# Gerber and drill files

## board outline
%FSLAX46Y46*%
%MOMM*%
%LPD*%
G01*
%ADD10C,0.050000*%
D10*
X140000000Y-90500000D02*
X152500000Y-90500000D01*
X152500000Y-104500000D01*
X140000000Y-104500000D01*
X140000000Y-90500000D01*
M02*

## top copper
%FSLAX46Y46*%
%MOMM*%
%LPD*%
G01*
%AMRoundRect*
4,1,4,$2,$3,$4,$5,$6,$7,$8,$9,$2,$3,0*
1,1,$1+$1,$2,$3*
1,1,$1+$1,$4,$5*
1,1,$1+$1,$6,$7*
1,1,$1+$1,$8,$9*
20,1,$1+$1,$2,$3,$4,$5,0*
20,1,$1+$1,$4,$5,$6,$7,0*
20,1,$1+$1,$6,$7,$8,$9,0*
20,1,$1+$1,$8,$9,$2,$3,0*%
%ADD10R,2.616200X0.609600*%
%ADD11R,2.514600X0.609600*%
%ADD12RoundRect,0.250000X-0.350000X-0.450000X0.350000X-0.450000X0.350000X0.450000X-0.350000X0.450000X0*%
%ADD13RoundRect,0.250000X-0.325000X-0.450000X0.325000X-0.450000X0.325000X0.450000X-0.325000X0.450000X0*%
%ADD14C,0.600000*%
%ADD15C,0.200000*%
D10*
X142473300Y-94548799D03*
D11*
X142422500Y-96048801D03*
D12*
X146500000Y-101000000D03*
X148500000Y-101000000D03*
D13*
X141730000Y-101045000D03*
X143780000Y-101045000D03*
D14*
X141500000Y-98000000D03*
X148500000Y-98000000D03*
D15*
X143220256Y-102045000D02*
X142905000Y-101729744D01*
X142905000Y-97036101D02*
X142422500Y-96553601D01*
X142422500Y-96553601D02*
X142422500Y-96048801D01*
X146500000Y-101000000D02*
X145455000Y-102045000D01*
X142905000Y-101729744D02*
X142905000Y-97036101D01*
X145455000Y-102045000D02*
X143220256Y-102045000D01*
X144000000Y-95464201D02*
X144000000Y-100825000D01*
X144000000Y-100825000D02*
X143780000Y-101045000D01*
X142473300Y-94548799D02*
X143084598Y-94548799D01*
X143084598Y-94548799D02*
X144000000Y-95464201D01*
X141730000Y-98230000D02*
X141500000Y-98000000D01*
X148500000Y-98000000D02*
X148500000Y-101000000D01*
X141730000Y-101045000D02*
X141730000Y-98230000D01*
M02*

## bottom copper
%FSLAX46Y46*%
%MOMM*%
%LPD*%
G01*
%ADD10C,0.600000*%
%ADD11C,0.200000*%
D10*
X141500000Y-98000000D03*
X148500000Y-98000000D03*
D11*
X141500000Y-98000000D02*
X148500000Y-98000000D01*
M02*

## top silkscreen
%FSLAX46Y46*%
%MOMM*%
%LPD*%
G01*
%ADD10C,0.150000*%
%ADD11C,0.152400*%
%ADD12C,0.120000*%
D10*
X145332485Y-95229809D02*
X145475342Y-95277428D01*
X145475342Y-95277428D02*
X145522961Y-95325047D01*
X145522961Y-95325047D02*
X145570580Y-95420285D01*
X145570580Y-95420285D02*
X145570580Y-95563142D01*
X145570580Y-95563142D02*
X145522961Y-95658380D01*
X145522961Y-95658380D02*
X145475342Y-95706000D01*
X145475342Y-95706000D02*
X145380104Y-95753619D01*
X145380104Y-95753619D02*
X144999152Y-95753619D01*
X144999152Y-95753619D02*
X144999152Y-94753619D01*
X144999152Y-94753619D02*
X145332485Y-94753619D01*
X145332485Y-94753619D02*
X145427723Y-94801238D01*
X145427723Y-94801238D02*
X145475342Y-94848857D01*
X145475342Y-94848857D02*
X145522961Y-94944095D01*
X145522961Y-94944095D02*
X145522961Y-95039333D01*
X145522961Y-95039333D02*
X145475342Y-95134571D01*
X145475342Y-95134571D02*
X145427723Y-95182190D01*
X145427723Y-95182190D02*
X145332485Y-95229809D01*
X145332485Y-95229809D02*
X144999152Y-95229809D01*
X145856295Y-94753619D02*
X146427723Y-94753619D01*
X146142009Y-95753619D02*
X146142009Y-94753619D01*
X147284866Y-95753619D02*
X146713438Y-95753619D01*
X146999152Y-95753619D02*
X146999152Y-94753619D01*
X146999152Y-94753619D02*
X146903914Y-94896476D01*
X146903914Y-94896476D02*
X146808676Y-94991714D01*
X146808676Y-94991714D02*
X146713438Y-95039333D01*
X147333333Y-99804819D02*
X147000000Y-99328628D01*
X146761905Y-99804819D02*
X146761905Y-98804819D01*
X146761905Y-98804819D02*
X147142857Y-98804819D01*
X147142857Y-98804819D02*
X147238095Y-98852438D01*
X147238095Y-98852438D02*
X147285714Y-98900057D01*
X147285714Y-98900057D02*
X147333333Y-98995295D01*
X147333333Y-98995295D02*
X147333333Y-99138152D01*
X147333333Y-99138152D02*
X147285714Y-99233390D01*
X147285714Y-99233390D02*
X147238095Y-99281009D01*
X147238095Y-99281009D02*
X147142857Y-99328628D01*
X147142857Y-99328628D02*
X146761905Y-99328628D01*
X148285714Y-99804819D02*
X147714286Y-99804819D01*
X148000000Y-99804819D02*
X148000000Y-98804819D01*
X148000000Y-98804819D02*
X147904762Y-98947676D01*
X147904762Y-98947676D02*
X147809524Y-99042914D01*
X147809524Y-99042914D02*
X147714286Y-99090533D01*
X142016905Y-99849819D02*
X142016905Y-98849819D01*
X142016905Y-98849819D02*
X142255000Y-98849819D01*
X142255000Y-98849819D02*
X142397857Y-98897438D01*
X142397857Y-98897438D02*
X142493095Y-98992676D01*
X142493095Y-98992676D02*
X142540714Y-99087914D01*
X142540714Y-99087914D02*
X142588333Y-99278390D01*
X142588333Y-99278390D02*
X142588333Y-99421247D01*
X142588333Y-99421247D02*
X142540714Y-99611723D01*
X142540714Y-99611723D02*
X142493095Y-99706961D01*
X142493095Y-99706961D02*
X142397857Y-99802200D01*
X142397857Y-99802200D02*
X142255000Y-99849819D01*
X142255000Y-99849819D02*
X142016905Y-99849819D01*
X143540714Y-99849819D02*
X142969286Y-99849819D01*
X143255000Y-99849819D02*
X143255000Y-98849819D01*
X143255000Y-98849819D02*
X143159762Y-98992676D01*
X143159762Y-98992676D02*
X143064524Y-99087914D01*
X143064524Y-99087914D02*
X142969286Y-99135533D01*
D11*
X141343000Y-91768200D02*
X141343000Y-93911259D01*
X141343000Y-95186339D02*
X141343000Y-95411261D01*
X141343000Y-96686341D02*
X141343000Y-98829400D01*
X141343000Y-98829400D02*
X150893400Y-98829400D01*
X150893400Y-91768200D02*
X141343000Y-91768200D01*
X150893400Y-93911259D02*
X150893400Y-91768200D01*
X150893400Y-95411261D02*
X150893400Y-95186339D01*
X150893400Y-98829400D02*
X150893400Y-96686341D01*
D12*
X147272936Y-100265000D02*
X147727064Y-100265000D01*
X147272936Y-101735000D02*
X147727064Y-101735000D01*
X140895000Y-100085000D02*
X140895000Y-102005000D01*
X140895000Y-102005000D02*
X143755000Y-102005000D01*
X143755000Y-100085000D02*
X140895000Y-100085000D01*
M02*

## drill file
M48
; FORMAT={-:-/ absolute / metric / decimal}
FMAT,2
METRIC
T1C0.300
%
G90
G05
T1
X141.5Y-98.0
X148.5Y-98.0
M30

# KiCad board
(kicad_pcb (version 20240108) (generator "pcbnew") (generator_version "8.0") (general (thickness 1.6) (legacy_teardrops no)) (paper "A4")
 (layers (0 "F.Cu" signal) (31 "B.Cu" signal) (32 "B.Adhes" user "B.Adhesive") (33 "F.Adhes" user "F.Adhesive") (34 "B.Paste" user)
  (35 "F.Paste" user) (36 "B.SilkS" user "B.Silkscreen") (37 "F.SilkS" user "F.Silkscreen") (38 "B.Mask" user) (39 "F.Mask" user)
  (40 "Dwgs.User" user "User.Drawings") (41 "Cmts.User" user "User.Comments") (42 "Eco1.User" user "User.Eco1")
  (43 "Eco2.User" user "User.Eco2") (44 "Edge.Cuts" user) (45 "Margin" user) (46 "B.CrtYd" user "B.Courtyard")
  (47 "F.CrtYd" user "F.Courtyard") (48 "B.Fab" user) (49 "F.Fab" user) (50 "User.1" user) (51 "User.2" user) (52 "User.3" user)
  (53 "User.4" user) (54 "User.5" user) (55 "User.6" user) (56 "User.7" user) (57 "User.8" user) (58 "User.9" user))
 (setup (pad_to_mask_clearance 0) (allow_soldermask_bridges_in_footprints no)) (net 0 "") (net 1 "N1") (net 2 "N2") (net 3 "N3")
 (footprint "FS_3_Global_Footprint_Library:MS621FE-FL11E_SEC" (layer "F.Cu") (at 146.1182 95.2988)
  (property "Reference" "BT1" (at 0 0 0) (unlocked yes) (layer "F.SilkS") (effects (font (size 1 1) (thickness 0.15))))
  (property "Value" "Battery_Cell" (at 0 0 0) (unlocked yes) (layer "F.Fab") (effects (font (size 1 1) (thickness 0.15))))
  (fp_line (start -4.7752 -3.5306) (end -4.7752 -1.387541) (stroke (width 0.1524) (type solid)) (layer "F.SilkS"))
  (fp_line (start -4.7752 -0.112461) (end -4.7752 0.112461) (stroke (width 0.1524) (type solid)) (layer "F.SilkS"))
  (fp_line (start -4.7752 1.387541) (end -4.7752 3.5306) (stroke (width 0.1524) (type solid)) (layer "F.SilkS"))
  (fp_line (start -4.7752 3.5306) (end 4.7752 3.5306) (stroke (width 0.1524) (type solid)) (layer "F.SilkS"))
  (fp_line (start 4.7752 -3.5306) (end -4.7752 -3.5306) (stroke (width 0.1524) (type solid)) (layer "F.SilkS"))
  (fp_line (start 4.7752 -1.387541) (end 4.7752 -3.5306) (stroke (width 0.1524) (type solid)) (layer "F.SilkS"))
  (fp_line (start 4.7752 0.112461) (end 4.7752 -0.112461) (stroke (width 0.1524) (type solid)) (layer "F.SilkS"))
  (fp_line (start 4.7752 3.5306) (end 4.7752 1.387541) (stroke (width 0.1524) (type solid)) (layer "F.SilkS"))
  (pad "1" smd rect (at -3.6449 -0.750001) (size 2.6162 0.6096) (layers "F.Cu" "F.Paste" "F.Mask") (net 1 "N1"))
  (pad "2" smd rect (at -3.6957 0.750001) (size 2.5146 0.6096) (layers "F.Cu" "F.Paste" "F.Mask") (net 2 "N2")))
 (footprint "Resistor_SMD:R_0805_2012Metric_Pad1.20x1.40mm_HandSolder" (layer "F.Cu") (at 147.5 101)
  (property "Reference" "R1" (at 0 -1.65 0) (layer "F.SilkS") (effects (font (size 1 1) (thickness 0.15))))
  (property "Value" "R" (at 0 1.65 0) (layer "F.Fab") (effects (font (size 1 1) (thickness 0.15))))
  (fp_line (start -0.227064 -0.735) (end 0.227064 -0.735) (stroke (width 0.12) (type solid)) (layer "F.SilkS"))
  (fp_line (start -0.227064 0.735) (end 0.227064 0.735) (stroke (width 0.12) (type solid)) (layer "F.SilkS"))
  (pad "1" smd roundrect (at -1 0) (size 1.2 1.4) (layers "F.Cu" "F.Paste" "F.Mask") (roundrect_rratio 0.208333) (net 2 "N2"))
  (pad "2" smd roundrect (at 1 0) (size 1.2 1.4) (layers "F.Cu" "F.Paste" "F.Mask") (roundrect_rratio 0.208333) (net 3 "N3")))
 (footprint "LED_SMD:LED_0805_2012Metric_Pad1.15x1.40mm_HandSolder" (layer "F.Cu") (at 142.755 101.045)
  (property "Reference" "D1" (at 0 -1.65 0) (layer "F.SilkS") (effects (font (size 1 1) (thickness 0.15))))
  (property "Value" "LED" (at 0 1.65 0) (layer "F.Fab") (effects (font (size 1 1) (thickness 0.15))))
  (fp_line (start -1.86 -0.96) (end -1.86 0.96) (stroke (width 0.12) (type solid)) (layer "F.SilkS"))
  (fp_line (start -1.86 0.96) (end 1 0.96) (stroke (width 0.12) (type solid)) (layer "F.SilkS"))
  (fp_line (start 1 -0.96) (end -1.86 -0.96) (stroke (width 0.12) (type solid)) (layer "F.SilkS"))
  (pad "1" smd roundrect (at -1.025 0) (size 1.15 1.4) (layers "F.Cu" "F.Paste" "F.Mask") (roundrect_rratio 0.217391) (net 3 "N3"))
  (pad "2" smd roundrect (at 1.025 0) (size 1.15 1.4) (layers "F.Cu" "F.Paste" "F.Mask") (roundrect_rratio 0.217391) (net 1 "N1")))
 (gr_rect (start 140 90.5) (end 152.5 104.5) (stroke (width 0.05) (type default)) (fill none) (layer "Edge.Cuts"))
 (segment (start 143.220256 102.045) (end 142.905 101.729744) (width 0.2) (layer "F.Cu") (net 2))
 (segment (start 142.905 97.036101) (end 142.4225 96.553601) (width 0.2) (layer "F.Cu") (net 2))
 (segment (start 142.4225 96.553601) (end 142.4225 96.048801) (width 0.2) (layer "F.Cu") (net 2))
 (segment (start 146.5 101) (end 145.455 102.045) (width 0.2) (layer "F.Cu") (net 2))
 (segment (start 142.905 101.729744) (end 142.905 97.036101) (width 0.2) (layer "F.Cu") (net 2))
 (segment (start 145.455 102.045) (end 143.220256 102.045) (width 0.2) (layer "F.Cu") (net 2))
 (segment (start 144 95.464201) (end 144 100.825) (width 0.2) (layer "F.Cu") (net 1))
 (segment (start 144 100.825) (end 143.78 101.045) (width 0.2) (layer "F.Cu") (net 1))
 (segment (start 142.4733 94.548799) (end 143.084598 94.548799) (width 0.2) (layer "F.Cu") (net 1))
 (segment (start 143.084598 94.548799) (end 144 95.464201) (width 0.2) (layer "F.Cu") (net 1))
 (segment (start 141.73 98.23) (end 141.5 98) (width 0.2) (layer "F.Cu") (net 3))
 (segment (start 148.5 98) (end 148.5 101) (width 0.2) (layer "F.Cu") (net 3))
 (segment (start 141.73 101.045) (end 141.73 98.23) (width 0.2) (layer "F.Cu") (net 3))
 (via (at 141.5 98) (size 0.6) (drill 0.3) (layers "F.Cu" "B.Cu") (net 3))
 (via (at 148.5 98) (size 0.6) (drill 0.3) (layers "F.Cu" "B.Cu") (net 3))
 (segment (start 141.5 98) (end 148.5 98) (width 0.2) (layer "B.Cu") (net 3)))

